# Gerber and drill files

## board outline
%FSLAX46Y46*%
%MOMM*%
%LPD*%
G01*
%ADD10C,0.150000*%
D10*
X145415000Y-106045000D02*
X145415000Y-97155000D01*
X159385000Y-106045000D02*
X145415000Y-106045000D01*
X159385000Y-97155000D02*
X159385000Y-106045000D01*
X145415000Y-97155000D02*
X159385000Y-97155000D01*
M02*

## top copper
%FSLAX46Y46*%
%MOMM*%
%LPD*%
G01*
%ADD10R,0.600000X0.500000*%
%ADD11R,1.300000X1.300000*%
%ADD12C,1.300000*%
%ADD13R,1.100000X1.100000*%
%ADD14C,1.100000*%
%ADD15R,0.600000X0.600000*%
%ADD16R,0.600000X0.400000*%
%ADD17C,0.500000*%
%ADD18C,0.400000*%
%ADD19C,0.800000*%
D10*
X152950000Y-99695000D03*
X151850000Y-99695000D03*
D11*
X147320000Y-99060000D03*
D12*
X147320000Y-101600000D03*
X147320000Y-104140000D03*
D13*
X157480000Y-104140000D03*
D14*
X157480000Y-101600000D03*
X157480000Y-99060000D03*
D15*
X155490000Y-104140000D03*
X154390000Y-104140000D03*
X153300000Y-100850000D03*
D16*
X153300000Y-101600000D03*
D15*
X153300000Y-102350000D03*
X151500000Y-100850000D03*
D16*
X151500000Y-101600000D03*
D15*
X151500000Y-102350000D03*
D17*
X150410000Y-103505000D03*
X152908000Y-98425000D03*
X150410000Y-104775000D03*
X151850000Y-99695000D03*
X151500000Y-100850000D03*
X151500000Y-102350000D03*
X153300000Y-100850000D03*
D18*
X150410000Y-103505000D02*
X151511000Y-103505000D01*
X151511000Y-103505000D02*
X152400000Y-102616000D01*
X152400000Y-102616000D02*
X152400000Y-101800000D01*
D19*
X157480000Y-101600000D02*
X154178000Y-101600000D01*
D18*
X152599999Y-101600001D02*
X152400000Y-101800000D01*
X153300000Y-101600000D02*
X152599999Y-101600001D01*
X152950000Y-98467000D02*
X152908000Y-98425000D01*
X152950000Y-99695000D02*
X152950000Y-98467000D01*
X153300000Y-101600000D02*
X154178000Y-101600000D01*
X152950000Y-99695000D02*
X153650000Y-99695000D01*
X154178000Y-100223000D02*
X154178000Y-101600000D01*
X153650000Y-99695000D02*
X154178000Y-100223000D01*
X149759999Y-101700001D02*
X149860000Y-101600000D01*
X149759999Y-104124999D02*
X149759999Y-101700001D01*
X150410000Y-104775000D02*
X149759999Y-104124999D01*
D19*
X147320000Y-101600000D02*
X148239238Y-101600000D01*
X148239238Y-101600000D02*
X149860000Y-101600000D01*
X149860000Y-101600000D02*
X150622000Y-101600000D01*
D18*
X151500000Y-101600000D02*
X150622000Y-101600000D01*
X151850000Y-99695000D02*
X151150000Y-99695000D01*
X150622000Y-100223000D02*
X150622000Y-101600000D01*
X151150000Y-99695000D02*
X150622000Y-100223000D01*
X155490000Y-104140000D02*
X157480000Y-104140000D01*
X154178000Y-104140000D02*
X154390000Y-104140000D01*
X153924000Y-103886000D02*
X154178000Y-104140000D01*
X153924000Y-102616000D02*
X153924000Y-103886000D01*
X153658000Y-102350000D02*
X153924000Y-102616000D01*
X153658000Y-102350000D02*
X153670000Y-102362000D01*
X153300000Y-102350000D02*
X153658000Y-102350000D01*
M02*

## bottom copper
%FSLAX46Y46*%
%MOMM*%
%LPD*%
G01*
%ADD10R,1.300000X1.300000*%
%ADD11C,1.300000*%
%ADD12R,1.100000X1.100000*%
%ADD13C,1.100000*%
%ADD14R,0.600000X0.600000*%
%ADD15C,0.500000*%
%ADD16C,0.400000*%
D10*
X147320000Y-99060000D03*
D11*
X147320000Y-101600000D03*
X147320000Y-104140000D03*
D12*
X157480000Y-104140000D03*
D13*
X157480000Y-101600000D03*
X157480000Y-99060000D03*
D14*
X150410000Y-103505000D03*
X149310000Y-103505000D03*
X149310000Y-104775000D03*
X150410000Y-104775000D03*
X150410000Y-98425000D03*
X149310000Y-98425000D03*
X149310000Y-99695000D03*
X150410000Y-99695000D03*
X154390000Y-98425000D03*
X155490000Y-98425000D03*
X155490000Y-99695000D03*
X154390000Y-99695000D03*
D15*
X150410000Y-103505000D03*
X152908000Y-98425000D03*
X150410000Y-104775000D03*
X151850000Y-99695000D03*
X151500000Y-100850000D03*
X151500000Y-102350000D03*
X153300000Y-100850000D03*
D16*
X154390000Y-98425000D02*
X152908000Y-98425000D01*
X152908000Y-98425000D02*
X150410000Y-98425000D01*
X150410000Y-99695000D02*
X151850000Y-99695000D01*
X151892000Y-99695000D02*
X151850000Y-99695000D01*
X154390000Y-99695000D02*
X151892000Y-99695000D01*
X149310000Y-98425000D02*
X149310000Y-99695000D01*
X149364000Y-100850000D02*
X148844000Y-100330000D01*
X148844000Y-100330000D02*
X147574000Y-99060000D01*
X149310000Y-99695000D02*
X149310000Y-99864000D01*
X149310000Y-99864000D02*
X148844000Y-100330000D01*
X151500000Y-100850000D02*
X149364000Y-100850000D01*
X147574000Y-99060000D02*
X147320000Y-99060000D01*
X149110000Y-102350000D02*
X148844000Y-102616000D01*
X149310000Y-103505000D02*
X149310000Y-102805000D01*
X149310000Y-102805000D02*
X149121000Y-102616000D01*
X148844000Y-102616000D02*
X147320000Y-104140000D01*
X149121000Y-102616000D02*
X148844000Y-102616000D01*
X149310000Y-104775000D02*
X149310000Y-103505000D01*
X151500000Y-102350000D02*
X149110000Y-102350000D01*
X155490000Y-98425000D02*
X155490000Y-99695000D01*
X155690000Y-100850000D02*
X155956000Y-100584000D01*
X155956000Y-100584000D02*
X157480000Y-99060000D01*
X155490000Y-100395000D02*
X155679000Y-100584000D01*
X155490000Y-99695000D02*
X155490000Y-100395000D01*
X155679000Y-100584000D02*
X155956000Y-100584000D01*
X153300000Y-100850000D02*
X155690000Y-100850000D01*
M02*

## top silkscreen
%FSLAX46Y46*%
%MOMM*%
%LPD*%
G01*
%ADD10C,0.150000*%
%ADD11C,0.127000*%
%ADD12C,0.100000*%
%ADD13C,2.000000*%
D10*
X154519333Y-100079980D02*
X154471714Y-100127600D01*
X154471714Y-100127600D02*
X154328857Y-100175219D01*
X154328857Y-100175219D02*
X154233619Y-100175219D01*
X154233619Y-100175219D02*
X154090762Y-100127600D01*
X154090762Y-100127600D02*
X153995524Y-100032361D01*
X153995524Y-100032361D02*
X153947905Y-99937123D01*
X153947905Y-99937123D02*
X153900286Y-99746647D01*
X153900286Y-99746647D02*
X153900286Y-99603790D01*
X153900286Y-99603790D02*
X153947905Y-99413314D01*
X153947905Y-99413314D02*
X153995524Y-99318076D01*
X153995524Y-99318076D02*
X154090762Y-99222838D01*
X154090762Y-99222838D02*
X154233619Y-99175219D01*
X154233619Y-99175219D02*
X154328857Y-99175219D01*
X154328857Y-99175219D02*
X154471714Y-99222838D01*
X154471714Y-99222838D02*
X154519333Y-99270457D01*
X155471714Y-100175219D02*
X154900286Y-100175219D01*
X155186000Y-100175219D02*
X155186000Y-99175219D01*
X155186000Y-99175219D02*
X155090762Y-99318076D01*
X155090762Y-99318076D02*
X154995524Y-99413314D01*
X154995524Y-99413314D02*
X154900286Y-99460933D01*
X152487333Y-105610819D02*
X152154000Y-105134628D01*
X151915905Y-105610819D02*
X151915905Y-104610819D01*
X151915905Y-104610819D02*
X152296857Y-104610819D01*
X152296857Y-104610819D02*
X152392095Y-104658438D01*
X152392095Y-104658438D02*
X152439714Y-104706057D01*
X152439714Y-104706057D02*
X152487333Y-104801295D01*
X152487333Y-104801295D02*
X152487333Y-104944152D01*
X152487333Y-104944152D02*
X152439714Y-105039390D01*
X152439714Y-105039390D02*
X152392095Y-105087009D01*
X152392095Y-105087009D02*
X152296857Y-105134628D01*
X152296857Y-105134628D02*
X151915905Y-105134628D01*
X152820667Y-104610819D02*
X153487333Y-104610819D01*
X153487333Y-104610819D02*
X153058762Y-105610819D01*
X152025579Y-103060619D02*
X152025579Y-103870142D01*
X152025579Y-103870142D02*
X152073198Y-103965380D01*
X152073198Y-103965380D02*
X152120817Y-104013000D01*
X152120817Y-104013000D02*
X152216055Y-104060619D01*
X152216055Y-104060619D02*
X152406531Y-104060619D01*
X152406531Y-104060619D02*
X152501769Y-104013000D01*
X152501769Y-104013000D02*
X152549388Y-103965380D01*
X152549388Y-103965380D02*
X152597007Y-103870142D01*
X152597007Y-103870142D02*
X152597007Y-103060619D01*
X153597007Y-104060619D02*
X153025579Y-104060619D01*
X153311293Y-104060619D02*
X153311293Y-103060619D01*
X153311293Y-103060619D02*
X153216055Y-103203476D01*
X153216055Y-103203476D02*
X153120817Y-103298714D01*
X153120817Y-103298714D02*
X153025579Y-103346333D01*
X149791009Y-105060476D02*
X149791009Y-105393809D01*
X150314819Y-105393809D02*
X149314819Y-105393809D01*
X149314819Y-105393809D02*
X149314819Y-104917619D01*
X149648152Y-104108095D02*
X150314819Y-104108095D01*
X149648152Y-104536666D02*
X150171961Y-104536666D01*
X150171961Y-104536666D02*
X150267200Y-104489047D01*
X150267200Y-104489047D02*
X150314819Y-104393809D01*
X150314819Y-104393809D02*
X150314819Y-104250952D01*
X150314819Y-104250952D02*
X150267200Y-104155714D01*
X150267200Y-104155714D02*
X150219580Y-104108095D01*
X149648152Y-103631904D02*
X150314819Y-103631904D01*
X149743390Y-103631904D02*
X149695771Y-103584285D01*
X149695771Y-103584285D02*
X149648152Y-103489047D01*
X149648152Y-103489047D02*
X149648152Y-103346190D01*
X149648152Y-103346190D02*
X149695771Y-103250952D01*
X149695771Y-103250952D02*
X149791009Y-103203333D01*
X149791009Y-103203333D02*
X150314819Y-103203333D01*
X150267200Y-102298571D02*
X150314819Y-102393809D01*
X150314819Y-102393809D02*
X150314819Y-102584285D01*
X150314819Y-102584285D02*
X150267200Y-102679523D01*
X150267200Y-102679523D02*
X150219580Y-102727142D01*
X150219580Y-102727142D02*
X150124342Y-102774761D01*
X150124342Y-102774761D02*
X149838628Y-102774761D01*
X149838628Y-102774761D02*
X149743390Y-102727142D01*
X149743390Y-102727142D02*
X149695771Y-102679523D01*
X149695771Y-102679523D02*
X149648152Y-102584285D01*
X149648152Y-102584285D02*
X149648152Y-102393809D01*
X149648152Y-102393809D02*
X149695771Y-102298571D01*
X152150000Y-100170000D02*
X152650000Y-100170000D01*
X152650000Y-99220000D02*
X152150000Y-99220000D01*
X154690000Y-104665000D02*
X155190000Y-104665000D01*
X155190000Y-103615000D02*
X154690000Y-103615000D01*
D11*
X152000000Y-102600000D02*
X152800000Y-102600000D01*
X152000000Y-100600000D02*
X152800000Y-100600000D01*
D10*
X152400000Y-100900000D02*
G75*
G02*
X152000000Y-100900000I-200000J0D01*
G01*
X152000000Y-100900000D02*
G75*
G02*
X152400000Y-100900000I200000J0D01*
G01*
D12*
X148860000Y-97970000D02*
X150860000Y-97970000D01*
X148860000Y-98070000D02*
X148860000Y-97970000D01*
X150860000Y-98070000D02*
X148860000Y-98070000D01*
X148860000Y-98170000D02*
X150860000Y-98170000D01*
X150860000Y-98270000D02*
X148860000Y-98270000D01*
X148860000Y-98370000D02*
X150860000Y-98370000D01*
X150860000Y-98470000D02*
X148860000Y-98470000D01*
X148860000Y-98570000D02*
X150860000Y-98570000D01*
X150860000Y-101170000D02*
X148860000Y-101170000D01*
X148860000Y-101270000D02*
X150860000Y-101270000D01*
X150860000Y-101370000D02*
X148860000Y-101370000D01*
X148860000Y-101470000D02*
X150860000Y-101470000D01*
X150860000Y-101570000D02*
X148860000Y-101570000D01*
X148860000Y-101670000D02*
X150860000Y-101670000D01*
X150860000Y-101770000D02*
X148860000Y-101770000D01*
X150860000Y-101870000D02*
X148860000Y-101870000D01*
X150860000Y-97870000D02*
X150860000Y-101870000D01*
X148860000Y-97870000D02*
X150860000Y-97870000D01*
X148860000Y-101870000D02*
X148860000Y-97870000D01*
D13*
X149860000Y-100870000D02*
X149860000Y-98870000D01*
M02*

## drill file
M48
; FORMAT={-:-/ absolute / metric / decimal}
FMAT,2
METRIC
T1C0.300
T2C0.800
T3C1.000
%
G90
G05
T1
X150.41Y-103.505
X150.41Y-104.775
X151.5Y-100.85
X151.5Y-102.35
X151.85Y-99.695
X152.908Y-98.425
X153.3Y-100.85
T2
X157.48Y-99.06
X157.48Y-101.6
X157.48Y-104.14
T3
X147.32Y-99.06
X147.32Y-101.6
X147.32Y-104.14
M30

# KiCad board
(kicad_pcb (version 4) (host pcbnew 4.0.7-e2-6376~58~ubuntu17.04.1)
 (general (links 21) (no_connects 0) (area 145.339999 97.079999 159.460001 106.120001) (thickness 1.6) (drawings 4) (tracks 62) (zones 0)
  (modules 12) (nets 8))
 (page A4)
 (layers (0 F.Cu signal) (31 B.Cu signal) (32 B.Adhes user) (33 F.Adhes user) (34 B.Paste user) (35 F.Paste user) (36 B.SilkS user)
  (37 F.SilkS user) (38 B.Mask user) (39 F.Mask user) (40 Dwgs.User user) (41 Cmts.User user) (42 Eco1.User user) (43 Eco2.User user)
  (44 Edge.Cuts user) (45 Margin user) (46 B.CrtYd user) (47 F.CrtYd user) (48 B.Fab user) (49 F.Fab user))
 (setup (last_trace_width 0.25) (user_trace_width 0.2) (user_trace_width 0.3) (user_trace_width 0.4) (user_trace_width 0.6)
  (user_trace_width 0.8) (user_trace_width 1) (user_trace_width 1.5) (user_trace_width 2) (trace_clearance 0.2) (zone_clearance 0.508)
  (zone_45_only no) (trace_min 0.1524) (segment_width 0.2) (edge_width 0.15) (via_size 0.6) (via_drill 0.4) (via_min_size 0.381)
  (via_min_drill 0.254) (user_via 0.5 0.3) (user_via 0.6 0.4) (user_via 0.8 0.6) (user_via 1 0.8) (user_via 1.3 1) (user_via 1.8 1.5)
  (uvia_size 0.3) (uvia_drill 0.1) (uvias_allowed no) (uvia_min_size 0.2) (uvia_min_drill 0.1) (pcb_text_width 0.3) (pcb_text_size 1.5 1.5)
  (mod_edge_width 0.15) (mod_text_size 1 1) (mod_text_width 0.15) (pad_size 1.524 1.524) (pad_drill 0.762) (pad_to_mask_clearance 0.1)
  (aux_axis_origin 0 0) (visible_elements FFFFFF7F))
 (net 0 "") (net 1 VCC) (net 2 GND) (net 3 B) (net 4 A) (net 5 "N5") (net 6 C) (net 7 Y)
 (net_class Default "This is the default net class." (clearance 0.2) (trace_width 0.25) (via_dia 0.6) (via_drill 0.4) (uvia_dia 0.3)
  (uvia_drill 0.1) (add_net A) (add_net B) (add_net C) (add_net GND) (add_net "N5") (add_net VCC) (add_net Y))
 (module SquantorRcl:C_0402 (layer F.Cu) (at 152.4 99.695 180)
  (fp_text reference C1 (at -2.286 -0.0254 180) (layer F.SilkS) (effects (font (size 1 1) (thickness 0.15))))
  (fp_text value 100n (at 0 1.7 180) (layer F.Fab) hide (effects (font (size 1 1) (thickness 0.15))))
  (fp_line (start 0.25 -0.475) (end -0.25 -0.475) (layer F.SilkS) (width 0.15))
  (fp_line (start -0.25 0.475) (end 0.25 0.475) (layer F.SilkS) (width 0.15))
  (pad 1 smd rect (at -0.55 0 180) (size 0.6 0.5) (layers F.Cu F.Paste F.Mask) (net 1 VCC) (solder_mask_margin 0.1))
  (pad 2 smd rect (at 0.55 0 180) (size 0.6 0.5) (layers F.Cu F.Paste F.Mask) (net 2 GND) (solder_mask_margin 0.1)))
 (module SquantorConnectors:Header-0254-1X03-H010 (layer B.Cu) (at 147.32 101.6 270)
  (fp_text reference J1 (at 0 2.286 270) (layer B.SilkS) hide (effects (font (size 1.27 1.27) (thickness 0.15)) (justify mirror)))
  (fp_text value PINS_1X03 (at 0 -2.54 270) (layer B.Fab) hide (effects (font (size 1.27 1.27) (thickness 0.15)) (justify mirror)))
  (pad 1 thru_hole rect (at -2.54 0 90) (size 1.3 1.3) (drill 1) (layers *.Cu *.Mask) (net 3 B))
  (pad 2 thru_hole circle (at 0 0 90) (size 1.3 1.3) (drill 1) (layers *.Cu *.Mask) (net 2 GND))
  (pad 3 thru_hole circle (at 2.54 0 90) (size 1.3 1.3) (drill 1) (layers *.Cu *.Mask) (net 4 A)))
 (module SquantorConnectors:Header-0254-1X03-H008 (layer B.Cu) (at 157.48 101.6 90)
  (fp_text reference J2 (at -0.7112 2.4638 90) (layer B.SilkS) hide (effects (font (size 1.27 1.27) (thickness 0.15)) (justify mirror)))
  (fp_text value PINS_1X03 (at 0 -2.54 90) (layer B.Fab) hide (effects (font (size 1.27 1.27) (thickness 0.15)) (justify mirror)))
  (pad 1 thru_hole rect (at -2.54 0 270) (size 1.1 1.1) (drill 0.8) (layers *.Cu *.Mask) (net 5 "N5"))
  (pad 2 thru_hole circle (at 0 0 270) (size 1.1 1.1) (drill 0.8) (layers *.Cu *.Mask) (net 1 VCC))
  (pad 3 thru_hole circle (at 2.54 0 270) (size 1.1 1.1) (drill 0.8) (layers *.Cu *.Mask) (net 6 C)))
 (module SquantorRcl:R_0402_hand (layer B.Cu) (at 149.86 103.505 180)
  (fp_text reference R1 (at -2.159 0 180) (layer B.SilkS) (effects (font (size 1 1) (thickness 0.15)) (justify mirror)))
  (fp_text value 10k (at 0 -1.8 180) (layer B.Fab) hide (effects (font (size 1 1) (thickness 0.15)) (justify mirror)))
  (pad 1 smd rect (at -0.55 0 180) (size 0.6 0.6) (layers B.Cu B.Paste B.Mask) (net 1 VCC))
  (pad 2 smd rect (at 0.55 0 180) (size 0.6 0.6) (layers B.Cu B.Paste B.Mask) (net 4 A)))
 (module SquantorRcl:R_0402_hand (layer B.Cu) (at 149.86 104.775)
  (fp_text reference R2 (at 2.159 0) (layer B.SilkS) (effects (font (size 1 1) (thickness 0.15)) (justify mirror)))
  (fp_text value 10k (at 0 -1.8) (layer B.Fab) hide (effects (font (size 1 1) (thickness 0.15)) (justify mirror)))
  (pad 1 smd rect (at -0.55 0) (size 0.6 0.6) (layers B.Cu B.Paste B.Mask) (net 4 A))
  (pad 2 smd rect (at 0.55 0) (size 0.6 0.6) (layers B.Cu B.Paste B.Mask) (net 2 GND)))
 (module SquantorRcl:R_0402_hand (layer B.Cu) (at 149.86 98.425 180)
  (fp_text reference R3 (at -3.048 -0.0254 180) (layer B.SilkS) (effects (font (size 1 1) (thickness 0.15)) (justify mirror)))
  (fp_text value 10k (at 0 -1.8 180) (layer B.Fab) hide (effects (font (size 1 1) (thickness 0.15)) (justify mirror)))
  (pad 1 smd rect (at -0.55 0 180) (size 0.6 0.6) (layers B.Cu B.Paste B.Mask) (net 1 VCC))
  (pad 2 smd rect (at 0.55 0 180) (size 0.6 0.6) (layers B.Cu B.Paste B.Mask) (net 3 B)))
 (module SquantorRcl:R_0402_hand (layer B.Cu) (at 149.86 99.695)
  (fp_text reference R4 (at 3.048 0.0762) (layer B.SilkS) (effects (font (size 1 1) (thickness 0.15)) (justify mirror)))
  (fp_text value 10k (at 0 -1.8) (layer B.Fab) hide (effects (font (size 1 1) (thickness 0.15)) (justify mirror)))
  (pad 1 smd rect (at -0.55 0) (size 0.6 0.6) (layers B.Cu B.Paste B.Mask) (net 3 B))
  (pad 2 smd rect (at 0.55 0) (size 0.6 0.6) (layers B.Cu B.Paste B.Mask) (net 2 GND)))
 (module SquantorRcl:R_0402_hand (layer B.Cu) (at 154.94 98.425)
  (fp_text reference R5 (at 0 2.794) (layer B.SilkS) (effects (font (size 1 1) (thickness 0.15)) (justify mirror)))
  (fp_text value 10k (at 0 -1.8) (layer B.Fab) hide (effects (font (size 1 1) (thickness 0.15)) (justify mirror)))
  (pad 1 smd rect (at -0.55 0) (size 0.6 0.6) (layers B.Cu B.Paste B.Mask) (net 1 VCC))
  (pad 2 smd rect (at 0.55 0) (size 0.6 0.6) (layers B.Cu B.Paste B.Mask) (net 6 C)))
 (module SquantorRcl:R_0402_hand (layer B.Cu) (at 154.94 99.695 180)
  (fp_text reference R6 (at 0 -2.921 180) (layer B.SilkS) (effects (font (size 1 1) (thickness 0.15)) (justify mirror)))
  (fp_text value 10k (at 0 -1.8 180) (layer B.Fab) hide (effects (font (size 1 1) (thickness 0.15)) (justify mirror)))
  (pad 1 smd rect (at -0.55 0 180) (size 0.6 0.6) (layers B.Cu B.Paste B.Mask) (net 6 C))
  (pad 2 smd rect (at 0.55 0 180) (size 0.6 0.6) (layers B.Cu B.Paste B.Mask) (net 2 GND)))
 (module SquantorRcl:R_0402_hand (layer F.Cu) (at 154.94 104.14 180)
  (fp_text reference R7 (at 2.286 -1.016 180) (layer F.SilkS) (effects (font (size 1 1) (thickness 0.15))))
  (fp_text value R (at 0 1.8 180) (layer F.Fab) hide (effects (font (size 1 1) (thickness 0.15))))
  (fp_line (start 0.25 -0.525) (end -0.25 -0.525) (layer F.SilkS) (width 0.15))
  (fp_line (start -0.25 0.525) (end 0.25 0.525) (layer F.SilkS) (width 0.15))
  (pad 1 smd rect (at -0.55 0 180) (size 0.6 0.6) (layers F.Cu F.Paste F.Mask) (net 5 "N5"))
  (pad 2 smd rect (at 0.55 0 180) (size 0.6 0.6) (layers F.Cu F.Paste F.Mask) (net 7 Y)))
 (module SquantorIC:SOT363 (layer F.Cu) (at 152.4 101.6 270)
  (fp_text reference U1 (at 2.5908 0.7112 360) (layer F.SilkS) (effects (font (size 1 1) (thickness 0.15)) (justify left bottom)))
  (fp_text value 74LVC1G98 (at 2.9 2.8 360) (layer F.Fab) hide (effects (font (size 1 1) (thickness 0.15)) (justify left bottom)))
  (fp_line (start 1 0.4) (end 1 -0.4) (layer F.SilkS) (width 0.127))
  (fp_line (start -1 0.4) (end -1 -0.4) (layer F.SilkS) (width 0.127))
  (fp_circle (center -0.7 0.2) (end -0.5 0.2) (layer F.SilkS) (width 0.15))
  (pad 6 smd rect (at -0.75 -0.9 270) (size 0.6 0.6) (layers F.Cu F.Paste F.Mask) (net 6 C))
  (pad 5 smd rect (at 0 -0.9 270) (size 0.4 0.6) (layers F.Cu F.Paste F.Mask) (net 1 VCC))
  (pad 4 smd rect (at 0.75 -0.9 270) (size 0.6 0.6) (layers F.Cu F.Paste F.Mask) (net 7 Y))
  (pad 1 smd rect (at -0.75 0.9 270) (size 0.6 0.6) (layers F.Cu F.Paste F.Mask) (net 3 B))
  (pad 2 smd rect (at 0 0.9 270) (size 0.4 0.6) (layers F.Cu F.Paste F.Mask) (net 2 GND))
  (pad 3 smd rect (at 0.75 0.9 270) (size 0.6 0.6) (layers F.Cu F.Paste F.Mask) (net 4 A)))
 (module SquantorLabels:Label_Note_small (layer F.Cu) (at 149.86 102.87 90)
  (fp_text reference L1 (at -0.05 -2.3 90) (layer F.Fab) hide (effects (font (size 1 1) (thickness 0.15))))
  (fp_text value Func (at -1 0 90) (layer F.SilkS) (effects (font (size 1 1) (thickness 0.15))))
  (fp_line (start 4.9 -1) (end 4.9 1) (layer F.SilkS) (width 0.1))
  (fp_line (start 4.8 -1) (end 4.9 -1) (layer F.SilkS) (width 0.1))
  (fp_line (start 4.8 1) (end 4.8 -1) (layer F.SilkS) (width 0.1))
  (fp_line (start 4.7 -1) (end 4.7 1) (layer F.SilkS) (width 0.1))
  (fp_line (start 4.6 1) (end 4.6 -1) (layer F.SilkS) (width 0.1))
  (fp_line (start 4.5 -1) (end 4.5 1) (layer F.SilkS) (width 0.1))
  (fp_line (start 4.4 1) (end 4.4 -1) (layer F.SilkS) (width 0.1))
  (fp_line (start 4.3 -1) (end 4.3 1) (layer F.SilkS) (width 0.1))
  (fp_line (start 1.7 1) (end 1.7 -1) (layer F.SilkS) (width 0.1))
  (fp_line (start 1.6 -1) (end 1.6 1) (layer F.SilkS) (width 0.1))
  (fp_line (start 1.5 1) (end 1.5 -1) (layer F.SilkS) (width 0.1))
  (fp_line (start 1.4 -1) (end 1.4 1) (layer F.SilkS) (width 0.1))
  (fp_line (start 1.3 1) (end 1.3 -1) (layer F.SilkS) (width 0.1))
  (fp_line (start 1.2 -1) (end 1.2 1) (layer F.SilkS) (width 0.1))
  (fp_line (start 1.1 1) (end 1.1 -1) (layer F.SilkS) (width 0.1)) (fp_line (start 1 1) (end 1 -1) (layer F.SilkS) (width 0.1))
  (fp_line (start 5 1) (end 1 1) (layer F.SilkS) (width 0.1)) (fp_line (start 5 -1) (end 5 1) (layer F.SilkS) (width 0.1))
  (fp_line (start 1 -1) (end 5 -1) (layer F.SilkS) (width 0.1)) (fp_line (start 2 0) (end 4 0) (layer F.SilkS) (width 2)))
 (gr_line (start 145.415 106.045) (end 145.415 97.155) (angle 90) (layer Edge.Cuts) (width 0.15))
 (gr_line (start 159.385 106.045) (end 145.415 106.045) (angle 90) (layer Edge.Cuts) (width 0.15))
 (gr_line (start 159.385 97.155) (end 159.385 106.045) (angle 90) (layer Edge.Cuts) (width 0.15))
 (gr_line (start 145.415 97.155) (end 159.385 97.155) (angle 90) (layer Edge.Cuts) (width 0.15))
 (segment (start 150.41 103.505) (end 151.511 103.505) (width 0.4) (layer F.Cu) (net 1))
 (segment (start 151.511 103.505) (end 152.4 102.616) (width 0.4) (layer F.Cu) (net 1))
 (segment (start 152.4 102.616) (end 152.4 101.8) (width 0.4) (layer F.Cu) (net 1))
 (via (at 150.41 103.505) (size 0.5) (drill 0.3) (layers F.Cu B.Cu) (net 1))
 (segment (start 157.48 101.6) (end 154.178 101.6) (width 0.8) (layer F.Cu) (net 1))
 (segment (start 152.599999 101.600001) (end 152.4 101.8) (width 0.4) (layer F.Cu) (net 1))
 (segment (start 153.3 101.6) (end 152.599999 101.600001) (width 0.4) (layer F.Cu) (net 1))
 (segment (start 154.39 98.425) (end 152.908 98.425) (width 0.4) (layer B.Cu) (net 1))
 (segment (start 152.908 98.425) (end 150.41 98.425) (width 0.4) (layer B.Cu) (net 1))
 (segment (start 152.95 98.467) (end 152.908 98.425) (width 0.4) (layer F.Cu) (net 1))
 (via (at 152.908 98.425) (size 0.5) (drill 0.3) (layers F.Cu B.Cu) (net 1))
 (segment (start 152.95 99.695) (end 152.95 98.467) (width 0.4) (layer F.Cu) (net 1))
 (segment (start 153.3 101.6) (end 154.178 101.6) (width 0.4) (layer F.Cu) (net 1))
 (segment (start 152.95 99.695) (end 153.65 99.695) (width 0.4) (layer F.Cu) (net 1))
 (segment (start 154.178 100.223) (end 154.178 101.6) (width 0.4) (layer F.Cu) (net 1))
 (segment (start 153.65 99.695) (end 154.178 100.223) (width 0.4) (layer F.Cu) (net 1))
 (segment (start 149.759999 101.700001) (end 149.86 101.6) (width 0.4) (layer F.Cu) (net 2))
 (segment (start 149.759999 104.124999) (end 149.759999 101.700001) (width 0.4) (layer F.Cu) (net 2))
 (segment (start 150.41 104.775) (end 149.759999 104.124999) (width 0.4) (layer F.Cu) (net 2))
 (segment (start 147.32 101.6) (end 148.239238 101.6) (width 0.8) (layer F.Cu) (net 2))
 (segment (start 148.239238 101.6) (end 149.86 101.6) (width 0.8) (layer F.Cu) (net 2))
 (segment (start 149.86 101.6) (end 150.622 101.6) (width 0.8) (layer F.Cu) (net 2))
 (via (at 150.41 104.775) (size 0.5) (drill 0.3) (layers F.Cu B.Cu) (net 2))
 (segment (start 150.41 99.695) (end 151.85 99.695) (width 0.4) (layer B.Cu) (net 2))
 (segment (start 151.892 99.695) (end 151.85 99.695) (width 0.4) (layer B.Cu) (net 2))
 (via (at 151.85 99.695) (size 0.5) (drill 0.3) (layers F.Cu B.Cu) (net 2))
 (segment (start 154.39 99.695) (end 151.892 99.695) (width 0.4) (layer B.Cu) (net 2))
 (segment (start 151.5 101.6) (end 150.622 101.6) (width 0.4) (layer F.Cu) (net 2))
 (segment (start 151.85 99.695) (end 151.15 99.695) (width 0.4) (layer F.Cu) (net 2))
 (segment (start 150.622 100.223) (end 150.622 101.6) (width 0.4) (layer F.Cu) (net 2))
 (segment (start 151.15 99.695) (end 150.622 100.223) (width 0.4) (layer F.Cu) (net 2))
 (segment (start 149.31 98.425) (end 149.31 99.695) (width 0.4) (layer B.Cu) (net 3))
 (segment (start 149.364 100.85) (end 148.844 100.33) (width 0.4) (layer B.Cu) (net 3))
 (segment (start 148.844 100.33) (end 147.574 99.06) (width 0.4) (layer B.Cu) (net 3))
 (segment (start 149.31 99.695) (end 149.31 99.864) (width 0.4) (layer B.Cu) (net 3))
 (segment (start 149.31 99.864) (end 148.844 100.33) (width 0.4) (layer B.Cu) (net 3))
 (segment (start 151.5 100.85) (end 149.364 100.85) (width 0.4) (layer B.Cu) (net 3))
 (segment (start 147.574 99.06) (end 147.32 99.06) (width 0.4) (layer B.Cu) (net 3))
 (via (at 151.5 100.85) (size 0.5) (drill 0.3) (layers F.Cu B.Cu) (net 3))
 (segment (start 149.11 102.35) (end 148.844 102.616) (width 0.4) (layer B.Cu) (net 4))
 (segment (start 149.31 103.505) (end 149.31 102.805) (width 0.4) (layer B.Cu) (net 4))
 (segment (start 149.31 102.805) (end 149.121 102.616) (width 0.4) (layer B.Cu) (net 4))
 (segment (start 148.844 102.616) (end 147.32 104.14) (width 0.4) (layer B.Cu) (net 4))
 (segment (start 149.121 102.616) (end 148.844 102.616) (width 0.4) (layer B.Cu) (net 4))
 (segment (start 149.31 104.775) (end 149.31 103.505) (width 0.4) (layer B.Cu) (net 4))
 (segment (start 151.5 102.35) (end 149.11 102.35) (width 0.4) (layer B.Cu) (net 4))
 (via (at 151.5 102.35) (size 0.5) (drill 0.3) (layers F.Cu B.Cu) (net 4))
 (segment (start 155.49 104.14) (end 157.48 104.14) (width 0.4) (layer F.Cu) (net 5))
 (segment (start 155.49 98.425) (end 155.49 99.695) (width 0.4) (layer B.Cu) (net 6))
 (segment (start 155.69 100.85) (end 155.956 100.584) (width 0.4) (layer B.Cu) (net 6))
 (segment (start 155.956 100.584) (end 157.48 99.06) (width 0.4) (layer B.Cu) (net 6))
 (segment (start 155.49 100.395) (end 155.679 100.584) (width 0.4) (layer B.Cu) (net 6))
 (segment (start 155.49 99.695) (end 155.49 100.395) (width 0.4) (layer B.Cu) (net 6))
 (segment (start 155.679 100.584) (end 155.956 100.584) (width 0.4) (layer B.Cu) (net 6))
 (segment (start 153.3 100.85) (end 155.69 100.85) (width 0.4) (layer B.Cu) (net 6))
 (via (at 153.3 100.85) (size 0.5) (drill 0.3) (layers F.Cu B.Cu) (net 6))
 (segment (start 154.178 104.14) (end 154.39 104.14) (width 0.4) (layer F.Cu) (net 7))
 (segment (start 153.924 103.886) (end 154.178 104.14) (width 0.4) (layer F.Cu) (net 7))
 (segment (start 153.924 102.616) (end 153.924 103.886) (width 0.4) (layer F.Cu) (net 7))
 (segment (start 153.658 102.35) (end 153.924 102.616) (width 0.4) (layer F.Cu) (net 7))
 (segment (start 153.658 102.35) (end 153.67 102.362) (width 0.4) (layer F.Cu) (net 7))
 (segment (start 153.3 102.35) (end 153.658 102.35) (width 0.4) (layer F.Cu) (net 7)))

